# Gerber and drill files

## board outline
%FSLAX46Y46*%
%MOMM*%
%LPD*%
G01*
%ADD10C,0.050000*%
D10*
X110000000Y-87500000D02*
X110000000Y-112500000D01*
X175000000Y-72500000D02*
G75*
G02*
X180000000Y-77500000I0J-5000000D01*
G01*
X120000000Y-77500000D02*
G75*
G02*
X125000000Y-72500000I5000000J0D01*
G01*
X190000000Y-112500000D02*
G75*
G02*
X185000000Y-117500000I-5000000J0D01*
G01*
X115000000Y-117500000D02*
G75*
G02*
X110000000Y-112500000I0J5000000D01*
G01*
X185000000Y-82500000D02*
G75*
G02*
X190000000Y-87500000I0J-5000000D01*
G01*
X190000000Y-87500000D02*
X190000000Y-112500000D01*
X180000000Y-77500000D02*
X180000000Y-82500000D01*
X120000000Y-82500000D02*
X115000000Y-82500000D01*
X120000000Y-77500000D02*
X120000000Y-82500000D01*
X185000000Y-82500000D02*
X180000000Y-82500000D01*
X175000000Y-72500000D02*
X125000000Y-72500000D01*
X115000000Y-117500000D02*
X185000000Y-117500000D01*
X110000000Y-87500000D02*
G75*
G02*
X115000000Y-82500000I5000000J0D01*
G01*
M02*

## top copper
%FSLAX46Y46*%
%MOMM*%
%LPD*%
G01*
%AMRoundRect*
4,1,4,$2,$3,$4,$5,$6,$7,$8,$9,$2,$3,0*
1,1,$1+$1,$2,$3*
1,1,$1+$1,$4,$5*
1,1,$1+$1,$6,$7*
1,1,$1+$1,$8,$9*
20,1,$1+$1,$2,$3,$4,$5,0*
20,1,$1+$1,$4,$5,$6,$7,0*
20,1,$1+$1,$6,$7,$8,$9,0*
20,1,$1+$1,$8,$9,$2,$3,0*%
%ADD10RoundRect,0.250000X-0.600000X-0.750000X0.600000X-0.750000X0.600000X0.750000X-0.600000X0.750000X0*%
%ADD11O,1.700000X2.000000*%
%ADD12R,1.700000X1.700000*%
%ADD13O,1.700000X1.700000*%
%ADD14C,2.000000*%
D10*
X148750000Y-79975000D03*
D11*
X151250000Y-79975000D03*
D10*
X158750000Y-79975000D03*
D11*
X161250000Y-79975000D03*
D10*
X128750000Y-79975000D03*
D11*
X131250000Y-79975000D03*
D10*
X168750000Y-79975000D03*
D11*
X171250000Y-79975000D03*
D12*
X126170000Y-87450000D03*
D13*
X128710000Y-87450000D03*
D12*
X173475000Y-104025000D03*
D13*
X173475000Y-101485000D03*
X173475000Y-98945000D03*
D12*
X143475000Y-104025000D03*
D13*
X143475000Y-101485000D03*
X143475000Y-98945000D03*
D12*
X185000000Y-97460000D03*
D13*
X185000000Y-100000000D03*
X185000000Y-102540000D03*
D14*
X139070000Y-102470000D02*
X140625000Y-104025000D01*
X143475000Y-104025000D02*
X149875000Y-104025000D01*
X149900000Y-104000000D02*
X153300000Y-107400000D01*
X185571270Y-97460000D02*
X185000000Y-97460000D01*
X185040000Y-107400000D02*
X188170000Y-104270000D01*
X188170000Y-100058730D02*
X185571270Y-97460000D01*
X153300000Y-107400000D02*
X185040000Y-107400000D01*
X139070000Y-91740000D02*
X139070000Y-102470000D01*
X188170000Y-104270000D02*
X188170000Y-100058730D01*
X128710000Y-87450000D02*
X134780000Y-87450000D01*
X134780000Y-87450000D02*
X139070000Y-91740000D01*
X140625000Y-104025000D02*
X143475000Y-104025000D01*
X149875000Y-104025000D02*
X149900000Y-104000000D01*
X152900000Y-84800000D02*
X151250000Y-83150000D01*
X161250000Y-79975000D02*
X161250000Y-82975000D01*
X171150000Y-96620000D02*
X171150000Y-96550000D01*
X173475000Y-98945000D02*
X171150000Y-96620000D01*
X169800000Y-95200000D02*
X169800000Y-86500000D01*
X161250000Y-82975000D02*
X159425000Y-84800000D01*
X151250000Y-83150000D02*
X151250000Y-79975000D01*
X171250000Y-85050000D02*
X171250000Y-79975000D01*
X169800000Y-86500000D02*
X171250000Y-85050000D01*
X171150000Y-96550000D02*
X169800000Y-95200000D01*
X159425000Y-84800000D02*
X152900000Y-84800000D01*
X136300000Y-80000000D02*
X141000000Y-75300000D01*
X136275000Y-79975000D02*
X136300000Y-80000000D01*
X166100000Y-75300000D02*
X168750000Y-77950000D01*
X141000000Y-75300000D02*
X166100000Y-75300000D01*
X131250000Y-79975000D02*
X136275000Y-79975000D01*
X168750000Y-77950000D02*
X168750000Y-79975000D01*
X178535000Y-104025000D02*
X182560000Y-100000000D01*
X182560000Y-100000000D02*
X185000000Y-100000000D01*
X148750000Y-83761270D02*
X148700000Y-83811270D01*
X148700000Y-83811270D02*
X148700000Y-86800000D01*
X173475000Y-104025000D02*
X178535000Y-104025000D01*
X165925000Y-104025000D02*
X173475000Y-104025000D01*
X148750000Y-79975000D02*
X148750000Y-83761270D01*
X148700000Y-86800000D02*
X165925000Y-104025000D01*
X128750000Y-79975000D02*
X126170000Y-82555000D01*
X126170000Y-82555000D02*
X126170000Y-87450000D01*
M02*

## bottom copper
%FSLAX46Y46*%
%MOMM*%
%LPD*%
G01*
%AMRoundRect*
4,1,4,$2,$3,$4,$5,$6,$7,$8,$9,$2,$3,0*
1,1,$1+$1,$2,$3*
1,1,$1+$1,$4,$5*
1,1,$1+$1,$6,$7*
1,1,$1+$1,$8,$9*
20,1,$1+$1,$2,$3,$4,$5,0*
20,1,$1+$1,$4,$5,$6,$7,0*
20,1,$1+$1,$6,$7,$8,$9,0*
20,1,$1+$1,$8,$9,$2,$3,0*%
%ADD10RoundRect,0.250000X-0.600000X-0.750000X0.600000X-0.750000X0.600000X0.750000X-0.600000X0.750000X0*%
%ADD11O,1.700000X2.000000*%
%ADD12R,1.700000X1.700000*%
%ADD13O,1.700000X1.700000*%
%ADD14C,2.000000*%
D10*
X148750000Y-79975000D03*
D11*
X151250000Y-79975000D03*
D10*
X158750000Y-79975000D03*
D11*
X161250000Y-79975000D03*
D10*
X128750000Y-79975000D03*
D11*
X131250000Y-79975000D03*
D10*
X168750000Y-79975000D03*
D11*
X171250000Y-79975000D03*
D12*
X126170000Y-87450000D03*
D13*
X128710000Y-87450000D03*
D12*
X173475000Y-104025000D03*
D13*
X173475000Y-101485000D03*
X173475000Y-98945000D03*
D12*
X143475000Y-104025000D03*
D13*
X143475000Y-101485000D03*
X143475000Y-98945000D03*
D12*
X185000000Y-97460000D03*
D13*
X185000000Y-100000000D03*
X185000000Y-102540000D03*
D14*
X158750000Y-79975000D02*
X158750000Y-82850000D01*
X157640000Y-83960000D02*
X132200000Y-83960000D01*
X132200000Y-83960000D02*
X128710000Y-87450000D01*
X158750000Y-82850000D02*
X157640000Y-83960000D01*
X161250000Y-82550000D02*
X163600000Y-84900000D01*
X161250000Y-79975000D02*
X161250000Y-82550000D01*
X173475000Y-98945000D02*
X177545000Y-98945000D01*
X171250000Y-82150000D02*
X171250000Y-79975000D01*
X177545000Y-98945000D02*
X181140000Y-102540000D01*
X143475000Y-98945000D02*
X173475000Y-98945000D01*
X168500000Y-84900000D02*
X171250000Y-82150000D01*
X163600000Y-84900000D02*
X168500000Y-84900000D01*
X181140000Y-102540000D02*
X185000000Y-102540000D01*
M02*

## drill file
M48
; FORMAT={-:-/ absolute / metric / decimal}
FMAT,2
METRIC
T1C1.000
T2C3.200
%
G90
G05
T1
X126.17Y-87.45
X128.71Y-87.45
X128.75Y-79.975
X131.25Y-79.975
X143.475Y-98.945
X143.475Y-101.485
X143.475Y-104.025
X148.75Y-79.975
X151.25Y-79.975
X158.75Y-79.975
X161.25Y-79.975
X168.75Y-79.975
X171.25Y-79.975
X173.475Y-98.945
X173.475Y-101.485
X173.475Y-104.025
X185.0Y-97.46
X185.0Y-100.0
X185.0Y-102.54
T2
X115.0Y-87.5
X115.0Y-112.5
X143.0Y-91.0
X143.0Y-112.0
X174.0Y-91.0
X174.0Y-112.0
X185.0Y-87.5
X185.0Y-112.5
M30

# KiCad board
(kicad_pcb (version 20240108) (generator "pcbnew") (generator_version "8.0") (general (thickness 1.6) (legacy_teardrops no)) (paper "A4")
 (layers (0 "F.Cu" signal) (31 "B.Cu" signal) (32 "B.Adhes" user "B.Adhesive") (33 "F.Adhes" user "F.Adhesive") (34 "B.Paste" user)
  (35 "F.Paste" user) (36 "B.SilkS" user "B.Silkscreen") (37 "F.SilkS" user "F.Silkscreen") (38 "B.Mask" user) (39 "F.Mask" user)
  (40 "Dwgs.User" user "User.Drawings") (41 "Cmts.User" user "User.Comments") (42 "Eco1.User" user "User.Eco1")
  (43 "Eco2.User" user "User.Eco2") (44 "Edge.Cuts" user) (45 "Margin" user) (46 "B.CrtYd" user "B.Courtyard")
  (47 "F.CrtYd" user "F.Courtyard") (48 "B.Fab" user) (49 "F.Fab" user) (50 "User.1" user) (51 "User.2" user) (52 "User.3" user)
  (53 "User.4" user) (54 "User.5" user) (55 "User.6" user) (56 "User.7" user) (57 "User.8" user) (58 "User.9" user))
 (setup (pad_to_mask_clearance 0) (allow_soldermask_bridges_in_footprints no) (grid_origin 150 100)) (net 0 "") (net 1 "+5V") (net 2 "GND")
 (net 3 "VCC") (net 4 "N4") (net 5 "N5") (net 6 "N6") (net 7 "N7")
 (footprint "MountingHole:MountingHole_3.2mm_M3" (layer "F.Cu") (at 143 91)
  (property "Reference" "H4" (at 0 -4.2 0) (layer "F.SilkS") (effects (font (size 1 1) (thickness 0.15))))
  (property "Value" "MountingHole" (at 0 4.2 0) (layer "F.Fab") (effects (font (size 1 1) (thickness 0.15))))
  (pad "" np_thru_hole circle (at 0 0) (size 3.2 3.2) (drill 3.2) (layers "*.Cu" "*.Mask")))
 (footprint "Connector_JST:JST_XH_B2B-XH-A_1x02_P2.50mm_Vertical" (layer "F.Cu") (at 148.75 79.975)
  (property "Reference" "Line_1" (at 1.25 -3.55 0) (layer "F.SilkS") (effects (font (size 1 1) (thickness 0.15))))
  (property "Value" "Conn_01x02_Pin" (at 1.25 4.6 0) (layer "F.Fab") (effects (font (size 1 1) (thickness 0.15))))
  (pad "1" thru_hole roundrect (at 0 0) (size 1.7 2) (drill 1) (layers "*.Cu" "*.Mask") (remove_unused_layers no)
   (roundrect_rratio 0.147059) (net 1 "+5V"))
  (pad "2" thru_hole oval (at 2.5 0) (size 1.7 2) (drill 1) (layers "*.Cu" "*.Mask") (remove_unused_layers no) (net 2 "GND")))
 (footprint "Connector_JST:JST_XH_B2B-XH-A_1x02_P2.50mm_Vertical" (layer "F.Cu") (at 158.75 79.975)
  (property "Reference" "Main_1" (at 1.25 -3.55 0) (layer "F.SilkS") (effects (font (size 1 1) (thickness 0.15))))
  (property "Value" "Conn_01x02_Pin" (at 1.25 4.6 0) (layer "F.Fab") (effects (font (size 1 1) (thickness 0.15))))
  (pad "1" thru_hole roundrect (at 0 0) (size 1.7 2) (drill 1) (layers "*.Cu" "*.Mask") (remove_unused_layers no)
   (roundrect_rratio 0.147059) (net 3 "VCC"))
  (pad "2" thru_hole oval (at 2.5 0) (size 1.7 2) (drill 1) (layers "*.Cu" "*.Mask") (remove_unused_layers no) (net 2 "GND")))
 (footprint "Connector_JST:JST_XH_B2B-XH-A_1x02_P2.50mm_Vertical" (layer "F.Cu") (at 128.75 79.975)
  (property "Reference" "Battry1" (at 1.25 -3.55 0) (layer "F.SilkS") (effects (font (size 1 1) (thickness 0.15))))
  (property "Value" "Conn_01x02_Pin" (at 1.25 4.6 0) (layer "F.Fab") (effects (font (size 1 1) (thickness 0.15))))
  (pad "1" thru_hole roundrect (at 0 0) (size 1.7 2) (drill 1) (layers "*.Cu" "*.Mask") (remove_unused_layers no)
   (roundrect_rratio 0.147059) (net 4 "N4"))
  (pad "2" thru_hole oval (at 2.5 0) (size 1.7 2) (drill 1) (layers "*.Cu" "*.Mask") (remove_unused_layers no) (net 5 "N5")))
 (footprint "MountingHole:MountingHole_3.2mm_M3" (layer "F.Cu") (at 115 112.5)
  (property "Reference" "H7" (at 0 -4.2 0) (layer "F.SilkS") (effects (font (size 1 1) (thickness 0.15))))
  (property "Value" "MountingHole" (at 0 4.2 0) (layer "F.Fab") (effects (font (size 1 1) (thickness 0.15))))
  (pad "" np_thru_hole circle (at 0 0) (size 3.2 3.2) (drill 3.2) (layers "*.Cu" "*.Mask")))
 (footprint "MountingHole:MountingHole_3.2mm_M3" (layer "F.Cu") (at 185 87.5)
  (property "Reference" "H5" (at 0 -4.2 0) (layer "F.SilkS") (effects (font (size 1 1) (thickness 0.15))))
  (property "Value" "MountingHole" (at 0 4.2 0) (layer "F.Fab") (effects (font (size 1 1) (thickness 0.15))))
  (pad "" np_thru_hole circle (at 0 0) (size 3.2 3.2) (drill 3.2) (layers "*.Cu" "*.Mask")))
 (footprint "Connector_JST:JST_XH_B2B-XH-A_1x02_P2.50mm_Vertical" (layer "F.Cu") (at 168.75 79.975)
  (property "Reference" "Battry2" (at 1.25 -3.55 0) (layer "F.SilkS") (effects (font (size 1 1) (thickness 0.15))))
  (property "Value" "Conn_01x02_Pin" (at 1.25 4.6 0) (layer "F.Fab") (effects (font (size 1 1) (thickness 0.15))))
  (pad "1" thru_hole roundrect (at 0 0) (size 1.7 2) (drill 1) (layers "*.Cu" "*.Mask") (remove_unused_layers no)
   (roundrect_rratio 0.147059) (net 5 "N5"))
  (pad "2" thru_hole oval (at 2.5 0) (size 1.7 2) (drill 1) (layers "*.Cu" "*.Mask") (remove_unused_layers no) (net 2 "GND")))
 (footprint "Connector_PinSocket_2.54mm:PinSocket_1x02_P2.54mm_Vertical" (layer "F.Cu") (at 126.17 87.45 90)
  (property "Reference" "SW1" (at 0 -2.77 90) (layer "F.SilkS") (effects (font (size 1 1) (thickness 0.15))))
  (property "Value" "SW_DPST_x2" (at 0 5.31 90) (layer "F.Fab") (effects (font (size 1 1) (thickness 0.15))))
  (pad "1" thru_hole rect (at 0 0 90) (size 1.7 1.7) (drill 1) (layers "*.Cu" "*.Mask") (remove_unused_layers no) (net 4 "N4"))
  (pad "2" thru_hole oval (at 0 2.54 90) (size 1.7 1.7) (drill 1) (layers "*.Cu" "*.Mask") (remove_unused_layers no) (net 3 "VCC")))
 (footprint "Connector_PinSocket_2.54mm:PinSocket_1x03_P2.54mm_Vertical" (layer "F.Cu") (at 173.475 104.025 180)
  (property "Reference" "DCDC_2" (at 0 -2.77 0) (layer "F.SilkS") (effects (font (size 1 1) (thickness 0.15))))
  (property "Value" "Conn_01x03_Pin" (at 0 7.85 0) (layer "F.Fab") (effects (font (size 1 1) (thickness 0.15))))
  (pad "1" thru_hole rect (at 0 0 180) (size 1.7 1.7) (drill 1) (layers "*.Cu" "*.Mask") (remove_unused_layers no) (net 1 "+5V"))
  (pad "2" thru_hole oval (at 0 2.54 180) (size 1.7 1.7) (drill 1) (layers "*.Cu" "*.Mask") (remove_unused_layers no) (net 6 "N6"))
  (pad "3" thru_hole oval (at 0 5.08 180) (size 1.7 1.7) (drill 1) (layers "*.Cu" "*.Mask") (remove_unused_layers no) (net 2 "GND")))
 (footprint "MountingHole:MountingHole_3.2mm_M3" (layer "F.Cu") (at 115 87.5)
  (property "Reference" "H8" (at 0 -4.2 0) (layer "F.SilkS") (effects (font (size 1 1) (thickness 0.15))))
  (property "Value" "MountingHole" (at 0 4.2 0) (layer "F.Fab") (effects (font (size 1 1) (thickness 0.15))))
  (pad "" np_thru_hole circle (at 0 0) (size 3.2 3.2) (drill 3.2) (layers "*.Cu" "*.Mask")))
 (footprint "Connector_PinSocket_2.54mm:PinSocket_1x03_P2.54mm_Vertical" (layer "F.Cu") (at 143.475 104.025 180)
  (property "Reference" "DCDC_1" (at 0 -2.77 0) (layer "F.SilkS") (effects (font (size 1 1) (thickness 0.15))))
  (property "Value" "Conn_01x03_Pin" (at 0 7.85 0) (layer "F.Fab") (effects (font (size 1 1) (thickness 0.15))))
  (pad "1" thru_hole rect (at 0 0 180) (size 1.7 1.7) (drill 1) (layers "*.Cu" "*.Mask") (remove_unused_layers no) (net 3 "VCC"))
  (pad "2" thru_hole oval (at 0 2.54 180) (size 1.7 1.7) (drill 1) (layers "*.Cu" "*.Mask") (remove_unused_layers no) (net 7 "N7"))
  (pad "3" thru_hole oval (at 0 5.08 180) (size 1.7 1.7) (drill 1) (layers "*.Cu" "*.Mask") (remove_unused_layers no) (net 2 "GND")))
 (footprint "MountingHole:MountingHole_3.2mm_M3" (layer "F.Cu") (at 143 112)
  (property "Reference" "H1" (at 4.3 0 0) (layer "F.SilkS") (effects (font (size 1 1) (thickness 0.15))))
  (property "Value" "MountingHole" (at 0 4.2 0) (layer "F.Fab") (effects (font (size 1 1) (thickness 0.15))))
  (pad "" np_thru_hole circle (at 0 0) (size 3.2 3.2) (drill 3.2) (layers "*.Cu" "*.Mask")))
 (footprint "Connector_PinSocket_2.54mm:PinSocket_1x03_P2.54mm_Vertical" (layer "F.Cu") (at 185 97.46)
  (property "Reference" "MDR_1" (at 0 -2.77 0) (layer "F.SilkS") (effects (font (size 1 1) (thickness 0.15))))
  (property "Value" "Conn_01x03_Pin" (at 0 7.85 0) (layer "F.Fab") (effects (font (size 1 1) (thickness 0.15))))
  (pad "1" thru_hole rect (at 0 0) (size 1.7 1.7) (drill 1) (layers "*.Cu" "*.Mask") (remove_unused_layers no) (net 3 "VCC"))
  (pad "2" thru_hole oval (at 0 2.54) (size 1.7 1.7) (drill 1) (layers "*.Cu" "*.Mask") (remove_unused_layers no) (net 1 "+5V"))
  (pad "3" thru_hole oval (at 0 5.08) (size 1.7 1.7) (drill 1) (layers "*.Cu" "*.Mask") (remove_unused_layers no) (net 2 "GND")))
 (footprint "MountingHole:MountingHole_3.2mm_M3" (layer "F.Cu") (at 174 91)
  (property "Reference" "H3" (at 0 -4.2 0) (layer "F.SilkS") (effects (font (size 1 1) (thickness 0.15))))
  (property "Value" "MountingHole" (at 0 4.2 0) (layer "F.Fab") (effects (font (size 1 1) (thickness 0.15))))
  (pad "" np_thru_hole circle (at 0 0) (size 3.2 3.2) (drill 3.2) (layers "*.Cu" "*.Mask")))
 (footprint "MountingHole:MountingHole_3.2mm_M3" (layer "F.Cu") (at 174 112)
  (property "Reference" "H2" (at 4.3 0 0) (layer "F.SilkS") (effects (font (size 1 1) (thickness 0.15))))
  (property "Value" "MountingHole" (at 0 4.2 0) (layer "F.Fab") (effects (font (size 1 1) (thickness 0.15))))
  (pad "" np_thru_hole circle (at 0 0) (size 3.2 3.2) (drill 3.2) (layers "*.Cu" "*.Mask")))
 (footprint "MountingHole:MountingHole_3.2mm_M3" (layer "F.Cu") (at 185 112.5)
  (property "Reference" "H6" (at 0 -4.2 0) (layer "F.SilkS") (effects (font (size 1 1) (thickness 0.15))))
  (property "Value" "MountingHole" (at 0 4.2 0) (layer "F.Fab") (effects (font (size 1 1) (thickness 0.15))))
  (pad "" np_thru_hole circle (at 0 0) (size 3.2 3.2) (drill 3.2) (layers "*.Cu" "*.Mask")))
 (gr_line (start 110 87.5) (end 110 112.5) (stroke (width 0.05) (type default)) (layer "Edge.Cuts"))
 (gr_arc (start 175 72.5) (mid 178.535534 73.964466) (end 180 77.5) (stroke (width 0.05) (type default)) (layer "Edge.Cuts"))
 (gr_arc (start 120 77.5) (mid 121.464466 73.964466) (end 125 72.5) (stroke (width 0.05) (type default)) (layer "Edge.Cuts"))
 (gr_arc (start 190 112.5) (mid 188.535534 116.035534) (end 185 117.5) (stroke (width 0.05) (type default)) (layer "Edge.Cuts"))
 (gr_arc (start 115 117.5) (mid 111.464466 116.035534) (end 110 112.5) (stroke (width 0.05) (type default)) (layer "Edge.Cuts"))
 (gr_arc (start 185 82.5) (mid 188.535534 83.964466) (end 190 87.5) (stroke (width 0.05) (type default)) (layer "Edge.Cuts"))
 (gr_line (start 190 87.5) (end 190 112.5) (stroke (width 0.05) (type default)) (layer "Edge.Cuts"))
 (gr_line (start 180 77.5) (end 180 82.5) (stroke (width 0.05) (type default)) (layer "Edge.Cuts"))
 (gr_line (start 120 82.5) (end 115 82.5) (stroke (width 0.05) (type default)) (layer "Edge.Cuts"))
 (gr_line (start 120 77.5) (end 120 82.5) (stroke (width 0.05) (type default)) (layer "Edge.Cuts"))
 (gr_line (start 185 82.5) (end 180 82.5) (stroke (width 0.05) (type default)) (layer "Edge.Cuts"))
 (gr_line (start 175 72.5) (end 125 72.5) (stroke (width 0.05) (type default)) (layer "Edge.Cuts"))
 (gr_line (start 115 117.5) (end 185 117.5) (stroke (width 0.05) (type default)) (layer "Edge.Cuts"))
 (gr_arc (start 110 87.5) (mid 111.464466 83.964466) (end 115 82.5) (stroke (width 0.05) (type default)) (layer "Edge.Cuts"))
 (segment (start 139.07 102.47) (end 140.625 104.025) (width 2) (layer "F.Cu") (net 3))
 (segment (start 143.475 104.025) (end 149.875 104.025) (width 2) (layer "F.Cu") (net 3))
 (segment (start 149.9 104) (end 153.3 107.4) (width 2) (layer "F.Cu") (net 3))
 (segment (start 185.57127 97.46) (end 185 97.46) (width 2) (layer "F.Cu") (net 3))
 (segment (start 185.04 107.4) (end 188.17 104.27) (width 2) (layer "F.Cu") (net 3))
 (segment (start 188.17 100.05873) (end 185.57127 97.46) (width 2) (layer "F.Cu") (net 3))
 (segment (start 153.3 107.4) (end 185.04 107.4) (width 2) (layer "F.Cu") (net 3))
 (segment (start 139.07 91.74) (end 139.07 102.47) (width 2) (layer "F.Cu") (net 3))
 (segment (start 188.17 104.27) (end 188.17 100.05873) (width 2) (layer "F.Cu") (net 3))
 (segment (start 128.71 87.45) (end 134.78 87.45) (width 2) (layer "F.Cu") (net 3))
 (segment (start 134.78 87.45) (end 139.07 91.74) (width 2) (layer "F.Cu") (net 3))
 (segment (start 140.625 104.025) (end 143.475 104.025) (width 2) (layer "F.Cu") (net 3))
 (segment (start 149.875 104.025) (end 149.9 104) (width 2) (layer "F.Cu") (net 3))
 (segment (start 158.75 79.975) (end 158.75 82.85) (width 2) (layer "B.Cu") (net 3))
 (segment (start 157.64 83.96) (end 132.2 83.96) (width 2) (layer "B.Cu") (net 3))
 (segment (start 132.2 83.96) (end 128.71 87.45) (width 2) (layer "B.Cu") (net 3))
 (segment (start 158.75 82.85) (end 157.64 83.96) (width 2) (layer "B.Cu") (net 3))
 (segment (start 152.9 84.8) (end 151.25 83.15) (width 2) (layer "F.Cu") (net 2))
 (segment (start 161.25 79.975) (end 161.25 82.975) (width 2) (layer "F.Cu") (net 2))
 (segment (start 171.15 96.62) (end 171.15 96.55) (width 2) (layer "F.Cu") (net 2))
 (segment (start 173.475 98.945) (end 171.15 96.62) (width 2) (layer "F.Cu") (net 2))
 (segment (start 169.8 95.2) (end 169.8 86.5) (width 2) (layer "F.Cu") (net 2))
 (segment (start 161.25 82.975) (end 159.425 84.8) (width 2) (layer "F.Cu") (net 2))
 (segment (start 151.25 83.15) (end 151.25 79.975) (width 2) (layer "F.Cu") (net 2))
 (segment (start 171.25 85.05) (end 171.25 79.975) (width 2) (layer "F.Cu") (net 2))
 (segment (start 169.8 86.5) (end 171.25 85.05) (width 2) (layer "F.Cu") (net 2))
 (segment (start 171.15 96.55) (end 169.8 95.2) (width 2) (layer "F.Cu") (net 2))
 (segment (start 159.425 84.8) (end 152.9 84.8) (width 2) (layer "F.Cu") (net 2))
 (segment (start 161.25 82.55) (end 163.6 84.9) (width 2) (layer "B.Cu") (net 2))
 (segment (start 161.25 79.975) (end 161.25 82.55) (width 2) (layer "B.Cu") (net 2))
 (segment (start 173.475 98.945) (end 177.545 98.945) (width 2) (layer "B.Cu") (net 2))
 (segment (start 171.25 82.15) (end 171.25 79.975) (width 2) (layer "B.Cu") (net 2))
 (segment (start 177.545 98.945) (end 181.14 102.54) (width 2) (layer "B.Cu") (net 2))
 (segment (start 143.475 98.945) (end 173.475 98.945) (width 2) (layer "B.Cu") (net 2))
 (segment (start 168.5 84.9) (end 171.25 82.15) (width 2) (layer "B.Cu") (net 2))
 (segment (start 163.6 84.9) (end 168.5 84.9) (width 2) (layer "B.Cu") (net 2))
 (segment (start 181.14 102.54) (end 185 102.54) (width 2) (layer "B.Cu") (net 2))
 (segment (start 136.3 80) (end 141 75.3) (width 2) (layer "F.Cu") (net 5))
 (segment (start 136.275 79.975) (end 136.3 80) (width 2) (layer "F.Cu") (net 5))
 (segment (start 166.1 75.3) (end 168.75 77.95) (width 2) (layer "F.Cu") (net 5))
 (segment (start 141 75.3) (end 166.1 75.3) (width 2) (layer "F.Cu") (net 5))
 (segment (start 131.25 79.975) (end 136.275 79.975) (width 2) (layer "F.Cu") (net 5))
 (segment (start 168.75 77.95) (end 168.75 79.975) (width 2) (layer "F.Cu") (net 5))
 (segment (start 178.535 104.025) (end 182.56 100) (width 2) (layer "F.Cu") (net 1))
 (segment (start 182.56 100) (end 185 100) (width 2) (layer "F.Cu") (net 1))
 (segment (start 148.75 83.76127) (end 148.7 83.81127) (width 2) (layer "F.Cu") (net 1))
 (segment (start 148.7 83.81127) (end 148.7 86.8) (width 2) (layer "F.Cu") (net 1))
 (segment (start 173.475 104.025) (end 178.535 104.025) (width 2) (layer "F.Cu") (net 1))
 (segment (start 165.925 104.025) (end 173.475 104.025) (width 2) (layer "F.Cu") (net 1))
 (segment (start 148.75 79.975) (end 148.75 83.76127) (width 2) (layer "F.Cu") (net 1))
 (segment (start 148.7 86.8) (end 165.925 104.025) (width 2) (layer "F.Cu") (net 1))
 (segment (start 128.75 79.975) (end 126.17 82.555) (width 2) (layer "F.Cu") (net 4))
 (segment (start 126.17 82.555) (end 126.17 87.45) (width 2) (layer "F.Cu") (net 4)))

